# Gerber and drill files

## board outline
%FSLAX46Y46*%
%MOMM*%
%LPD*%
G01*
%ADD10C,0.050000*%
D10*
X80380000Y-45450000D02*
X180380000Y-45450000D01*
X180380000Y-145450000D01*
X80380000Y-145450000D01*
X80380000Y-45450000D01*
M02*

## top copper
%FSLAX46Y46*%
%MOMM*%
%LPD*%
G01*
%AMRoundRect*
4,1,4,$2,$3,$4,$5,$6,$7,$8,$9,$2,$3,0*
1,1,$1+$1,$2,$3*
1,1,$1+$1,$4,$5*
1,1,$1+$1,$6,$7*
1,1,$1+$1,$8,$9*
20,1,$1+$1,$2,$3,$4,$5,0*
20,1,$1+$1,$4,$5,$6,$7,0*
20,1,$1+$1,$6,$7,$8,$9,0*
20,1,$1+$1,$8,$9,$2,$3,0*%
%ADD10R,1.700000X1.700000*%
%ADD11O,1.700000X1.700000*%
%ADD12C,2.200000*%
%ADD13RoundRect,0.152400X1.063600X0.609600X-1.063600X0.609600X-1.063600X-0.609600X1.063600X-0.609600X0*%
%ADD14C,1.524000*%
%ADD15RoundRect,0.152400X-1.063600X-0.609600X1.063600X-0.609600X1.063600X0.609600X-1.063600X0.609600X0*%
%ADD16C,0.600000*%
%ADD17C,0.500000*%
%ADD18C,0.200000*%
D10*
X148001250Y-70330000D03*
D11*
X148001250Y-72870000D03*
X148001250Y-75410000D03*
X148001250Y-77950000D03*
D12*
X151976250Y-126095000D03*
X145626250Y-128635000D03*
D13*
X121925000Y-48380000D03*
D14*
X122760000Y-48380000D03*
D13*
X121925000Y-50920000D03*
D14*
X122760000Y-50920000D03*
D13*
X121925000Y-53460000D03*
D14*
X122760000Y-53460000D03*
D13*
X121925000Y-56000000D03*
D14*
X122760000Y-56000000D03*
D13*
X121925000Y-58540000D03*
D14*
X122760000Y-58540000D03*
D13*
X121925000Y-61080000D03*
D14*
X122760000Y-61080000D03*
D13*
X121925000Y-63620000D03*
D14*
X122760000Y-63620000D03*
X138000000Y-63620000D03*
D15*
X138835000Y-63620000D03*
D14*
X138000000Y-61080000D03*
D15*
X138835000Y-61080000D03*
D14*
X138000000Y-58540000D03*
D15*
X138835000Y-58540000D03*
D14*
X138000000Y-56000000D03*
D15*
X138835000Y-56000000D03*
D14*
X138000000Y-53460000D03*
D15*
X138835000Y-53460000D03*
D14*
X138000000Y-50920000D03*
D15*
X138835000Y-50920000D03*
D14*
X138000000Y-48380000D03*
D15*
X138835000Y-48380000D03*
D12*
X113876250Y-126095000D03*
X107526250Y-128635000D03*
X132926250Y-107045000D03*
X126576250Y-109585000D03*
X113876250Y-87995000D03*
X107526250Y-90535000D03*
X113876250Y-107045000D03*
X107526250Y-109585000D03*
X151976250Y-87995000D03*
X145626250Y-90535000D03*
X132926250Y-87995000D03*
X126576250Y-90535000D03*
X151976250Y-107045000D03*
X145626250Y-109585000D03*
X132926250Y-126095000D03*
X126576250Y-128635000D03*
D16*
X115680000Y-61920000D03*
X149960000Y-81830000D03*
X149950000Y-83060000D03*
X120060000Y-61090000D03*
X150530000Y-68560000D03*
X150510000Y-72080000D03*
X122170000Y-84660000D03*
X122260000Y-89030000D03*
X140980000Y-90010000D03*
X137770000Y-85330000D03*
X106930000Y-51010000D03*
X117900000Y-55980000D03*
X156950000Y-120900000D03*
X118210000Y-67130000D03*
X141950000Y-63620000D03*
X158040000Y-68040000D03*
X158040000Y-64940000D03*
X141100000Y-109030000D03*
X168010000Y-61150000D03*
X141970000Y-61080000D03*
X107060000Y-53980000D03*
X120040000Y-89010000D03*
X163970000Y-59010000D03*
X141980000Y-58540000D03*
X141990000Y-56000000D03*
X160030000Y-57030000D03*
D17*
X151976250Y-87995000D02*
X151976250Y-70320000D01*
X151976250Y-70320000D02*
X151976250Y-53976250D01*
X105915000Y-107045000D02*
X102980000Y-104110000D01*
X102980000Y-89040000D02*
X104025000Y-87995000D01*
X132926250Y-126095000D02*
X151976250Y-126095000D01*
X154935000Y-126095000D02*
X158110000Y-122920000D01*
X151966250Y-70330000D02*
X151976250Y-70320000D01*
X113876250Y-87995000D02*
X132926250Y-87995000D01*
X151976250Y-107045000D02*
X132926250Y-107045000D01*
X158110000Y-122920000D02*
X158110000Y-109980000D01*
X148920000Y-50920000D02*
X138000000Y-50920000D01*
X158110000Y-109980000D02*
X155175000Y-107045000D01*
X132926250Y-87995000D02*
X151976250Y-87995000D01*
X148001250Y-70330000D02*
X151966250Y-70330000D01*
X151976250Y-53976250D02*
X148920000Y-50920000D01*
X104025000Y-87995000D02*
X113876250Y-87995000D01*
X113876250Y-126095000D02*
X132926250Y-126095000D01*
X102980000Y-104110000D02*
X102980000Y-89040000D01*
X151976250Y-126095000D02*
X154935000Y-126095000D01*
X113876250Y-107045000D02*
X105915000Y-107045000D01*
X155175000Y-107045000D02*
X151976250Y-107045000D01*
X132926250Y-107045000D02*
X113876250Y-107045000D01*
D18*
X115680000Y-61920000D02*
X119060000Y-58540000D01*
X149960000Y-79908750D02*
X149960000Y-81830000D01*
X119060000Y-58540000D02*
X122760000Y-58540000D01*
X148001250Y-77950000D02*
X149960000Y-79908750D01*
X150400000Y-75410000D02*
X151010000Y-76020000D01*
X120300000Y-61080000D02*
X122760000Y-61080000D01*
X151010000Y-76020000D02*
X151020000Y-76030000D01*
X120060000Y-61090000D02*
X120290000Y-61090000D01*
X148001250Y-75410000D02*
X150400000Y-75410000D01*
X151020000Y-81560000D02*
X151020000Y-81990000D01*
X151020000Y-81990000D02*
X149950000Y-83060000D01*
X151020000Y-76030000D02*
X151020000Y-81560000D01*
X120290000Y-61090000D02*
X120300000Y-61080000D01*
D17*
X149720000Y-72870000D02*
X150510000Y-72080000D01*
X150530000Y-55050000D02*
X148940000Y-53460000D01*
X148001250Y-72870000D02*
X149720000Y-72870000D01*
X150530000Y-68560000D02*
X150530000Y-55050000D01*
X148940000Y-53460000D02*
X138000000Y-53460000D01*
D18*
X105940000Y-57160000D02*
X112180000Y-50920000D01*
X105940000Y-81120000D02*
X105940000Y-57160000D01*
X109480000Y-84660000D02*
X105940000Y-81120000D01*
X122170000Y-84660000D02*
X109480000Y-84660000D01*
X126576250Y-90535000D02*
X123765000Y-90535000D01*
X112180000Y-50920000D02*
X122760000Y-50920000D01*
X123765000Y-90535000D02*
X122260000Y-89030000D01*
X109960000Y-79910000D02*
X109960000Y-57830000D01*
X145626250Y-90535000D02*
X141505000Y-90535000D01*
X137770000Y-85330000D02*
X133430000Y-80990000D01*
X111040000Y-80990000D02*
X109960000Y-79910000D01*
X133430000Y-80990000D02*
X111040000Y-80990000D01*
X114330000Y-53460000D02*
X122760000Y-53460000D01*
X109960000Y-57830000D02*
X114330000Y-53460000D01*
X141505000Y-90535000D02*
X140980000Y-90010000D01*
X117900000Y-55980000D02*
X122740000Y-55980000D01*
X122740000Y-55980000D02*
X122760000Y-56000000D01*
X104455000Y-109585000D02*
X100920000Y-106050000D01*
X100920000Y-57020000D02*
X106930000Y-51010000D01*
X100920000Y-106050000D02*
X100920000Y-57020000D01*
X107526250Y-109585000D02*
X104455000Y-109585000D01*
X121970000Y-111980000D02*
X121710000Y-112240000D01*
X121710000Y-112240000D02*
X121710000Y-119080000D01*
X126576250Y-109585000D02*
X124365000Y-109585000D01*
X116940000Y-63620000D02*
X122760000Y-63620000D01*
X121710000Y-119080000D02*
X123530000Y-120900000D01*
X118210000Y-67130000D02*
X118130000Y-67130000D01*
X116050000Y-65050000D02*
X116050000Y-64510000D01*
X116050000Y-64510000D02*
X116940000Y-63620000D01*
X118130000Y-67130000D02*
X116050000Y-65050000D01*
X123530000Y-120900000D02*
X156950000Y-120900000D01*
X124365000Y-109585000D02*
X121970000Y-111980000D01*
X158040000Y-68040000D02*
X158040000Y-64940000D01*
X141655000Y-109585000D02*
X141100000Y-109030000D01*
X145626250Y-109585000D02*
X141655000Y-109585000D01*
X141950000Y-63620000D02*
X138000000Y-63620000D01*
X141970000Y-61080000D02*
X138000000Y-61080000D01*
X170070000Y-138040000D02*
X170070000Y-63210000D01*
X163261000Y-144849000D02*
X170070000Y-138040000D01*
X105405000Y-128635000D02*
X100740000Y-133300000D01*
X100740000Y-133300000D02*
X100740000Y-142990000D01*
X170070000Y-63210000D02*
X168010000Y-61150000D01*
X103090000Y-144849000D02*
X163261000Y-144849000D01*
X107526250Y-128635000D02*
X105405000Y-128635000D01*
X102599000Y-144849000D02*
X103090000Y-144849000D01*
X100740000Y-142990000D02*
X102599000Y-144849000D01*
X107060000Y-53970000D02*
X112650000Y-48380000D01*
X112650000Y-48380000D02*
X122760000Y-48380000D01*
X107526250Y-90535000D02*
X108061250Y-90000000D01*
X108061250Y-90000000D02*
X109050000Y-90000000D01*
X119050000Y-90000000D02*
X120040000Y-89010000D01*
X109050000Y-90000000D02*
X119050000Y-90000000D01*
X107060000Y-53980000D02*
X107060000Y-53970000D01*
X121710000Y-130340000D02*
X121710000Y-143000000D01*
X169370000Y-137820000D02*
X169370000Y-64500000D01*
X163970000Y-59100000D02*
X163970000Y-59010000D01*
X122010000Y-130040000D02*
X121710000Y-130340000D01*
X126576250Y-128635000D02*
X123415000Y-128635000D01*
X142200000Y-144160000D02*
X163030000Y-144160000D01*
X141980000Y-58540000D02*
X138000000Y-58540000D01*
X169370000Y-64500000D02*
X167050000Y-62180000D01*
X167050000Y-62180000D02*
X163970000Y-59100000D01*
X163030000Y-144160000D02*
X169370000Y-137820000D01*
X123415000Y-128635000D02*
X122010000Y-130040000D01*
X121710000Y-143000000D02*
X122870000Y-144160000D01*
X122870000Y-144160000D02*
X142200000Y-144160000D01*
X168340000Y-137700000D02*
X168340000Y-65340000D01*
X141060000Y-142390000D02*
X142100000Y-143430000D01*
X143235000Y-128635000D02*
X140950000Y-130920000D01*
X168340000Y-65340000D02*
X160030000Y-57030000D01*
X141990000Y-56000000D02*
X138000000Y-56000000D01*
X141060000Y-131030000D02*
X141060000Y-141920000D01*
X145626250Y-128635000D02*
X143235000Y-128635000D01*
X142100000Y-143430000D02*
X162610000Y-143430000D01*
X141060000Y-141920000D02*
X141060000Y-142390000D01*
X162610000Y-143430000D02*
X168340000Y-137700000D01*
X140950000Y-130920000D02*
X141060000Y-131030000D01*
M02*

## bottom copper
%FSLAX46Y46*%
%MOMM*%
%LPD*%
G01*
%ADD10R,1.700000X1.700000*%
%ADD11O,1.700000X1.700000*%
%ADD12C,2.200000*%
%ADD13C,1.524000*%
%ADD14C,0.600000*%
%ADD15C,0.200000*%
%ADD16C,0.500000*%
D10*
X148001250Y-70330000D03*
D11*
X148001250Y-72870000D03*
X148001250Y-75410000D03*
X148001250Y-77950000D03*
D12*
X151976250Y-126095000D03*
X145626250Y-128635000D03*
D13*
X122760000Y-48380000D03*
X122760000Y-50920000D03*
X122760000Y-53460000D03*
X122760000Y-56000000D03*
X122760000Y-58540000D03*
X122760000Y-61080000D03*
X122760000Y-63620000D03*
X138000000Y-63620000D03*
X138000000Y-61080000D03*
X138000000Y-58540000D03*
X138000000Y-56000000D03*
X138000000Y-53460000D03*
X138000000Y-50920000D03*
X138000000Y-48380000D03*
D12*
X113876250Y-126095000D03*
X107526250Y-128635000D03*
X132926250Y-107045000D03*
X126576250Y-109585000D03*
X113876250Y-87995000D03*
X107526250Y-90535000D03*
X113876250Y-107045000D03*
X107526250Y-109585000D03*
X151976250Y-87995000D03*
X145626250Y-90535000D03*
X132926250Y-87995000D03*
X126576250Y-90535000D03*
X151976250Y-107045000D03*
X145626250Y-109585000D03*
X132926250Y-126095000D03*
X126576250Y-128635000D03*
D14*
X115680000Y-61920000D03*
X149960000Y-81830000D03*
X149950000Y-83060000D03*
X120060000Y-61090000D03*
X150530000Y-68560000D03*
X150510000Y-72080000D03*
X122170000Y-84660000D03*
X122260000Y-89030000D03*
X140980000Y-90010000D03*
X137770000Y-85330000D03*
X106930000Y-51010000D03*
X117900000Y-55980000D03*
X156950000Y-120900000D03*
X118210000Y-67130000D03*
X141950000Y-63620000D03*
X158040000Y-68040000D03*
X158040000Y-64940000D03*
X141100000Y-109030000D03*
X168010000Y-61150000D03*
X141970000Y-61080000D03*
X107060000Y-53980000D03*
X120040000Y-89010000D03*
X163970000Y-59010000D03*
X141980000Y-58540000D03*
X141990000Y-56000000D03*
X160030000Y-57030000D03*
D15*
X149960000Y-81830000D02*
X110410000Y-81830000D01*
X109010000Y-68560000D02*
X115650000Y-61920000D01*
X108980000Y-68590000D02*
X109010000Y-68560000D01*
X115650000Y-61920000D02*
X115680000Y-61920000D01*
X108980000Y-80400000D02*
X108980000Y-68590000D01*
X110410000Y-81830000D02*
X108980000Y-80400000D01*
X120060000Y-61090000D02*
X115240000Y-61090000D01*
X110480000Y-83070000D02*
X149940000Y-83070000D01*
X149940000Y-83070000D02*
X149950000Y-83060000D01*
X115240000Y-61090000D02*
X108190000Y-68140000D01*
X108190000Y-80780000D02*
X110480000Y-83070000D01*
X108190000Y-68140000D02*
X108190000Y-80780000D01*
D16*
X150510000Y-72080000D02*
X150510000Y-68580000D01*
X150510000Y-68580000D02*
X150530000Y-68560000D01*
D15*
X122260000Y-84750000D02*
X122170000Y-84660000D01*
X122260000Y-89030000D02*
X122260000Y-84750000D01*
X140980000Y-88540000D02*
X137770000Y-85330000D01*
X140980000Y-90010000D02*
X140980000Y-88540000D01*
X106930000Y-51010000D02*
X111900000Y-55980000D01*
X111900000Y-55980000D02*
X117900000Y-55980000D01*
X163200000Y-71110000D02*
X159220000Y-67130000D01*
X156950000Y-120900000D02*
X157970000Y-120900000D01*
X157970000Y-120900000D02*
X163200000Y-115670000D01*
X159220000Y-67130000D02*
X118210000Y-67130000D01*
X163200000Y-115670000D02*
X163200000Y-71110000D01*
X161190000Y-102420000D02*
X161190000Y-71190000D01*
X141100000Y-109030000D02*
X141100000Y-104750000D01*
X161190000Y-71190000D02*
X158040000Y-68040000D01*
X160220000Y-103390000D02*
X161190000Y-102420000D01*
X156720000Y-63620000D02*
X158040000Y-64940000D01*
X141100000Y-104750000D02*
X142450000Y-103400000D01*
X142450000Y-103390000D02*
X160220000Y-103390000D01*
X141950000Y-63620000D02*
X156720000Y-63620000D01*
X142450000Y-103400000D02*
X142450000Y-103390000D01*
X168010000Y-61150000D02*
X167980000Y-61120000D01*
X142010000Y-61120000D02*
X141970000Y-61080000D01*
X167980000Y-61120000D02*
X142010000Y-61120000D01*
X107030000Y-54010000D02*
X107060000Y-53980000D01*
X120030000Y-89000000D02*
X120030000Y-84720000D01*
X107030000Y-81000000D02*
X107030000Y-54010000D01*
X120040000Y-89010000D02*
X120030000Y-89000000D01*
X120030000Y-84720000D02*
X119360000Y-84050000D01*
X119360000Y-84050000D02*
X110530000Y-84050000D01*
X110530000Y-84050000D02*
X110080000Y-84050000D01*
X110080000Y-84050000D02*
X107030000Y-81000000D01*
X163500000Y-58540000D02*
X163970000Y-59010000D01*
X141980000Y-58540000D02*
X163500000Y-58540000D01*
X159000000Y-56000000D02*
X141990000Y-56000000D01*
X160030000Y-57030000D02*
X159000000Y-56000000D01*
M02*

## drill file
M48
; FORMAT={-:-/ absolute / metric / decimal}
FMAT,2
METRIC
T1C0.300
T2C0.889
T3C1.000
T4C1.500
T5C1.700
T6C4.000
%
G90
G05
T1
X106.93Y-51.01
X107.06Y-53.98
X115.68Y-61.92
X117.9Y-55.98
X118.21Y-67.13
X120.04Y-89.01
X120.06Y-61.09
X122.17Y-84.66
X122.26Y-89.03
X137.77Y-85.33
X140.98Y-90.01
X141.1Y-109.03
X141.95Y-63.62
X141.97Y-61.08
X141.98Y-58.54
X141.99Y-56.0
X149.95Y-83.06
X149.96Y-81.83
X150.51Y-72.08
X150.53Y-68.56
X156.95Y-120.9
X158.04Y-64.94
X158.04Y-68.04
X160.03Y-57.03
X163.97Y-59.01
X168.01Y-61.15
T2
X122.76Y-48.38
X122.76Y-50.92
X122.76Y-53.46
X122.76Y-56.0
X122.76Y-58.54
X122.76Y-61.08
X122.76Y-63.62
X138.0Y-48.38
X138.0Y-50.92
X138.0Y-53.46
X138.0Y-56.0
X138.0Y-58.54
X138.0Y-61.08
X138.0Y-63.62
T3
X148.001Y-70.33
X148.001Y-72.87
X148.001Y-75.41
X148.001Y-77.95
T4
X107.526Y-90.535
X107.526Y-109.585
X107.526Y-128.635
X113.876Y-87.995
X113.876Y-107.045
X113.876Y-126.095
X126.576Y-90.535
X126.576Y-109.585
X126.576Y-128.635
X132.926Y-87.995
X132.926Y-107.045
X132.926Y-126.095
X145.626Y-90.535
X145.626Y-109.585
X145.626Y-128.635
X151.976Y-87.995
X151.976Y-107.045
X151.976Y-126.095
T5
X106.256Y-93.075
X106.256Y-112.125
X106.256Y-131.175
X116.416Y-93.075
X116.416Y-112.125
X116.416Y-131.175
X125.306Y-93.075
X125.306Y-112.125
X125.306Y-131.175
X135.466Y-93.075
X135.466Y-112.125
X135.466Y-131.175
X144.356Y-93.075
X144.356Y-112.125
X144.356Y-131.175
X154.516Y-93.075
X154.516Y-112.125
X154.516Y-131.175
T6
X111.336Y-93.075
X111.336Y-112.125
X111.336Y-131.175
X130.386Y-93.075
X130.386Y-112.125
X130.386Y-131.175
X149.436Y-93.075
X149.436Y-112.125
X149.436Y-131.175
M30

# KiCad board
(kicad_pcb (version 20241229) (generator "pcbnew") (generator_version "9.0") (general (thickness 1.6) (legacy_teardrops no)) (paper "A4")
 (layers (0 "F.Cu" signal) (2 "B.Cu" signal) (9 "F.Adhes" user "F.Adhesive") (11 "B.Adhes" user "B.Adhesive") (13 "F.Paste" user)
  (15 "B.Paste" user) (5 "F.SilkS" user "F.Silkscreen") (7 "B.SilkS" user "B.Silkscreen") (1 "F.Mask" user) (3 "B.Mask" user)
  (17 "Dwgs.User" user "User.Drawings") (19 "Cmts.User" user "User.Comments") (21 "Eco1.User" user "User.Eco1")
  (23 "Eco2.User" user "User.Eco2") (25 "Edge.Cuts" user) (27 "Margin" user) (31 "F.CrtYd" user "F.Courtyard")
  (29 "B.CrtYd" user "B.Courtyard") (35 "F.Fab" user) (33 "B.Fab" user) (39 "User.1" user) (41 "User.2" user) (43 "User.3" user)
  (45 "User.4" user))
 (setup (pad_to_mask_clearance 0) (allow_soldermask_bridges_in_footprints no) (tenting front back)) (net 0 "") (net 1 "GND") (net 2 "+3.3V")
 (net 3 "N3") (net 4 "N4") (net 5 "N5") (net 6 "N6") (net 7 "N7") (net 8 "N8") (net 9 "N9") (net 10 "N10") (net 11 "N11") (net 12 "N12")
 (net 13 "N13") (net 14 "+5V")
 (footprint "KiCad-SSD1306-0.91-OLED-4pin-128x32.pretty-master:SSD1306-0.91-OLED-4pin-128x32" (layer "F.Cu") (at 111.50125 68.14)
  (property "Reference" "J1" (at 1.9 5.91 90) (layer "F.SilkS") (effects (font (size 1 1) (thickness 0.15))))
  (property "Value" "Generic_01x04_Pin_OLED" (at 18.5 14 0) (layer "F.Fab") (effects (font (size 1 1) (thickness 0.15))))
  (pad "1" thru_hole rect (at 36.5 2.19) (size 1.7 1.7) (drill 1) (layers "*.Cu" "*.Mask") (remove_unused_layers no) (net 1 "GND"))
  (pad "2" thru_hole oval (at 36.5 4.73) (size 1.7 1.7) (drill 1) (layers "*.Cu" "*.Mask") (remove_unused_layers no) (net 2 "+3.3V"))
  (pad "3" thru_hole oval (at 36.5 7.27) (size 1.7 1.7) (drill 1) (layers "*.Cu" "*.Mask") (remove_unused_layers no) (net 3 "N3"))
  (pad "4" thru_hole oval (at 36.5 9.81) (size 1.7 1.7) (drill 1) (layers "*.Cu" "*.Mask") (remove_unused_layers no) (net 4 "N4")))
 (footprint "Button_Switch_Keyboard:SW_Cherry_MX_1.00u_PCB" (layer "F.Cu") (at 151.97625 126.095)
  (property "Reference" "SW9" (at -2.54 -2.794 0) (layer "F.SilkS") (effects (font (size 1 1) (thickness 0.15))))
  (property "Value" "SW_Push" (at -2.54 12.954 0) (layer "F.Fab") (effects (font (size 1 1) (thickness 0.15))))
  (pad "" np_thru_hole circle (at -7.62 5.08) (size 1.7 1.7) (drill 1.7) (layers "*.Cu" "*.Mask"))
  (pad "" np_thru_hole circle (at -2.54 5.08) (size 4 4) (drill 4) (layers "*.Cu" "*.Mask"))
  (pad "" np_thru_hole circle (at 2.54 5.08) (size 1.7 1.7) (drill 1.7) (layers "*.Cu" "*.Mask"))
  (pad "1" thru_hole circle (at 0 0) (size 2.2 2.2) (drill 1.5) (layers "*.Cu" "*.Mask") (remove_unused_layers no) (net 1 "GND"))
  (pad "2" thru_hole circle (at -6.35 2.54) (size 2.2 2.2) (drill 1.5) (layers "*.Cu" "*.Mask") (remove_unused_layers no) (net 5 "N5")))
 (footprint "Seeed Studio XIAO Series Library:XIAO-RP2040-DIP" (layer "F.Cu") (at 130.38 56)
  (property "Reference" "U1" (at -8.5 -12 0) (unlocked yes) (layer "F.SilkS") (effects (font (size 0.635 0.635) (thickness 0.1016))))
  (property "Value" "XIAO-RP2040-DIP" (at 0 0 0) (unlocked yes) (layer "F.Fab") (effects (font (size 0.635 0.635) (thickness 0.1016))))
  (pad "1" smd roundrect (at -8.455 -7.62 180) (size 2.432 1.524) (layers "F.Cu" "F.Mask") (roundrect_rratio 0.1) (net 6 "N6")
   (thermal_bridge_angle 45))
  (pad "1" thru_hole circle (at -7.62 -7.62 180) (size 1.524 1.524) (drill 0.889) (layers "*.Cu" "*.Mask") (remove_unused_layers no)
   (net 6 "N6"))
  (pad "2" smd roundrect (at -8.455 -5.08 180) (size 2.432 1.524) (layers "F.Cu" "F.Mask") (roundrect_rratio 0.1) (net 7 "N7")
   (thermal_bridge_angle 45))
  (pad "2" thru_hole circle (at -7.62 -5.08 180) (size 1.524 1.524) (drill 0.889) (layers "*.Cu" "*.Mask") (remove_unused_layers no)
   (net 7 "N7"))
  (pad "3" smd roundrect (at -8.455 -2.54 180) (size 2.432 1.524) (layers "F.Cu" "F.Mask") (roundrect_rratio 0.1) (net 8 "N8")
   (thermal_bridge_angle 45))
  (pad "3" thru_hole circle (at -7.62 -2.54 180) (size 1.524 1.524) (drill 0.889) (layers "*.Cu" "*.Mask") (remove_unused_layers no)
   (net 8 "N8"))
  (pad "4" smd roundrect (at -8.455 0 180) (size 2.432 1.524) (layers "F.Cu" "F.Mask") (roundrect_rratio 0.1) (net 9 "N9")
   (thermal_bridge_angle 45))
  (pad "4" thru_hole circle (at -7.62 0 180) (size 1.524 1.524) (drill 0.889) (layers "*.Cu" "*.Mask") (remove_unused_layers no)
   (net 9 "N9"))
  (pad "5" smd roundrect (at -8.455 2.54 180) (size 2.432 1.524) (layers "F.Cu" "F.Mask") (roundrect_rratio 0.1) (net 4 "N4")
   (thermal_bridge_angle 45))
  (pad "5" thru_hole circle (at -7.62 2.54 180) (size 1.524 1.524) (drill 0.889) (layers "*.Cu" "*.Mask") (remove_unused_layers no)
   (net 4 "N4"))
  (pad "6" smd roundrect (at -8.455 5.08 180) (size 2.432 1.524) (layers "F.Cu" "F.Mask") (roundrect_rratio 0.1) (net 3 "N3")
   (thermal_bridge_angle 45))
  (pad "6" thru_hole circle (at -7.62 5.08 180) (size 1.524 1.524) (drill 0.889) (layers "*.Cu" "*.Mask") (remove_unused_layers no)
   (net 3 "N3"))
  (pad "7" smd roundrect (at -8.455 7.62 180) (size 2.432 1.524) (layers "F.Cu" "F.Mask") (roundrect_rratio 0.1) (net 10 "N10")
   (thermal_bridge_angle 45))
  (pad "7" thru_hole circle (at -7.62 7.62 180) (size 1.524 1.524) (drill 0.889) (layers "*.Cu" "*.Mask") (remove_unused_layers no)
   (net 10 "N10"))
  (pad "8" thru_hole circle (at 7.62 7.62) (size 1.524 1.524) (drill 0.889) (layers "*.Cu" "*.Mask") (remove_unused_layers no)
   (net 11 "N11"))
  (pad "8" smd roundrect (at 8.455 7.62) (size 2.432 1.524) (layers "F.Cu" "F.Mask") (roundrect_rratio 0.1) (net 11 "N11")
   (thermal_bridge_angle 45))
  (pad "9" thru_hole circle (at 7.62 5.08) (size 1.524 1.524) (drill 0.889) (layers "*.Cu" "*.Mask") (remove_unused_layers no)
   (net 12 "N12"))
  (pad "9" smd roundrect (at 8.455 5.08) (size 2.432 1.524) (layers "F.Cu" "F.Mask") (roundrect_rratio 0.1) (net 12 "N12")
   (thermal_bridge_angle 45))
  (pad "10" thru_hole circle (at 7.62 2.54) (size 1.524 1.524) (drill 0.889) (layers "*.Cu" "*.Mask") (remove_unused_layers no)
   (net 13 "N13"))
  (pad "10" smd roundrect (at 8.455 2.54) (size 2.432 1.524) (layers "F.Cu" "F.Mask") (roundrect_rratio 0.1) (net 13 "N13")
   (thermal_bridge_angle 45))
  (pad "11" thru_hole circle (at 7.62 0) (size 1.524 1.524) (drill 0.889) (layers "*.Cu" "*.Mask") (remove_unused_layers no) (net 5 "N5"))
  (pad "11" smd roundrect (at 8.455 0) (size 2.432 1.524) (layers "F.Cu" "F.Mask") (roundrect_rratio 0.1) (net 5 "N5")
   (thermal_bridge_angle 45))
  (pad "12" thru_hole circle (at 7.62 -2.54) (size 1.524 1.524) (drill 0.889) (layers "*.Cu" "*.Mask") (remove_unused_layers no)
   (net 2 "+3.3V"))
  (pad "12" smd roundrect (at 8.455 -2.54) (size 2.432 1.524) (layers "F.Cu" "F.Mask") (roundrect_rratio 0.1) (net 2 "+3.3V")
   (thermal_bridge_angle 45))
  (pad "13" thru_hole circle (at 7.62 -5.08) (size 1.524 1.524) (drill 0.889) (layers "*.Cu" "*.Mask") (remove_unused_layers no)
   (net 1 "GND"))
  (pad "13" smd roundrect (at 8.455 -5.08) (size 2.432 1.524) (layers "F.Cu" "F.Mask") (roundrect_rratio 0.1) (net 1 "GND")
   (thermal_bridge_angle 45))
  (pad "14" thru_hole circle (at 7.62 -7.62) (size 1.524 1.524) (drill 0.889) (layers "*.Cu" "*.Mask") (remove_unused_layers no)
   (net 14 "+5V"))
  (pad "14" smd roundrect (at 8.455 -7.62) (size 2.432 1.524) (layers "F.Cu" "F.Mask") (roundrect_rratio 0.1) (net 14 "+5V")
   (thermal_bridge_angle 45)))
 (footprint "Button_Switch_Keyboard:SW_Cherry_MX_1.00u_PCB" (layer "F.Cu") (at 113.87625 126.095)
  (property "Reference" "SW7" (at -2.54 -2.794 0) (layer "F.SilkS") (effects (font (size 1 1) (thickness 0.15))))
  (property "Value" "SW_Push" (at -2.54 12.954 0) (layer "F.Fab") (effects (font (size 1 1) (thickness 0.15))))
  (pad "" np_thru_hole circle (at -7.62 5.08) (size 1.7 1.7) (drill 1.7) (layers "*.Cu" "*.Mask"))
  (pad "" np_thru_hole circle (at -2.54 5.08) (size 4 4) (drill 4) (layers "*.Cu" "*.Mask"))
  (pad "" np_thru_hole circle (at 2.54 5.08) (size 1.7 1.7) (drill 1.7) (layers "*.Cu" "*.Mask"))
  (pad "1" thru_hole circle (at 0 0) (size 2.2 2.2) (drill 1.5) (layers "*.Cu" "*.Mask") (remove_unused_layers no) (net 1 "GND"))
  (pad "2" thru_hole circle (at -6.35 2.54) (size 2.2 2.2) (drill 1.5) (layers "*.Cu" "*.Mask") (remove_unused_layers no) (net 12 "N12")))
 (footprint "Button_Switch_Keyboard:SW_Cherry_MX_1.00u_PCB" (layer "F.Cu") (at 132.92625 107.045)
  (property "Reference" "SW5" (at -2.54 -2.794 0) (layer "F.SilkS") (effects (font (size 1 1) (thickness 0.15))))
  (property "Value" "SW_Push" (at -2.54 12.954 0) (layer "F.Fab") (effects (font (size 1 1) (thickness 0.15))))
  (pad "" np_thru_hole circle (at -7.62 5.08) (size 1.7 1.7) (drill 1.7) (layers "*.Cu" "*.Mask"))
  (pad "" np_thru_hole circle (at -2.54 5.08) (size 4 4) (drill 4) (layers "*.Cu" "*.Mask"))
  (pad "" np_thru_hole circle (at 2.54 5.08) (size 1.7 1.7) (drill 1.7) (layers "*.Cu" "*.Mask"))
  (pad "1" thru_hole circle (at 0 0) (size 2.2 2.2) (drill 1.5) (layers "*.Cu" "*.Mask") (remove_unused_layers no) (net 1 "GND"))
  (pad "2" thru_hole circle (at -6.35 2.54) (size 2.2 2.2) (drill 1.5) (layers "*.Cu" "*.Mask") (remove_unused_layers no) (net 10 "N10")))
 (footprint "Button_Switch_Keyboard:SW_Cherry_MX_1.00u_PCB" (layer "F.Cu") (at 113.87625 87.995)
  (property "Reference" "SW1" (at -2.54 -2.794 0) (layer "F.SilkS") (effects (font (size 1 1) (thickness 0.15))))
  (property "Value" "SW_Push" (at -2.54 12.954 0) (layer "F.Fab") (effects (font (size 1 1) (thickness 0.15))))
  (pad "" np_thru_hole circle (at -7.62 5.08) (size 1.7 1.7) (drill 1.7) (layers "*.Cu" "*.Mask"))
  (pad "" np_thru_hole circle (at -2.54 5.08) (size 4 4) (drill 4) (layers "*.Cu" "*.Mask"))
  (pad "" np_thru_hole circle (at 2.54 5.08) (size 1.7 1.7) (drill 1.7) (layers "*.Cu" "*.Mask"))
  (pad "1" thru_hole circle (at 0 0) (size 2.2 2.2) (drill 1.5) (layers "*.Cu" "*.Mask") (remove_unused_layers no) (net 1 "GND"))
  (pad "2" thru_hole circle (at -6.35 2.54) (size 2.2 2.2) (drill 1.5) (layers "*.Cu" "*.Mask") (remove_unused_layers no) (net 6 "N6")))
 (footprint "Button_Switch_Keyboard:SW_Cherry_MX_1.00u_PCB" (layer "F.Cu") (at 113.87625 107.045)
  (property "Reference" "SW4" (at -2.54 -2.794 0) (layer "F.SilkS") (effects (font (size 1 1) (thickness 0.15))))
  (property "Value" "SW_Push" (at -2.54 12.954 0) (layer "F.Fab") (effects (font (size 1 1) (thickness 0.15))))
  (pad "" np_thru_hole circle (at -7.62 5.08) (size 1.7 1.7) (drill 1.7) (layers "*.Cu" "*.Mask"))
  (pad "" np_thru_hole circle (at -2.54 5.08) (size 4 4) (drill 4) (layers "*.Cu" "*.Mask"))
  (pad "" np_thru_hole circle (at 2.54 5.08) (size 1.7 1.7) (drill 1.7) (layers "*.Cu" "*.Mask"))
  (pad "1" thru_hole circle (at 0 0) (size 2.2 2.2) (drill 1.5) (layers "*.Cu" "*.Mask") (remove_unused_layers no) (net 1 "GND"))
  (pad "2" thru_hole circle (at -6.35 2.54) (size 2.2 2.2) (drill 1.5) (layers "*.Cu" "*.Mask") (remove_unused_layers no) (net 9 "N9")))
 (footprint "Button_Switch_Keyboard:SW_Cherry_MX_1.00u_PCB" (layer "F.Cu") (at 151.97625 87.995)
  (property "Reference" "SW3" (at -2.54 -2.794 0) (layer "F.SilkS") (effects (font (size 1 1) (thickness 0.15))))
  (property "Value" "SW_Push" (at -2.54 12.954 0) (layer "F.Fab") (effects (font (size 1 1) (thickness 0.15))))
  (pad "" np_thru_hole circle (at -7.62 5.08) (size 1.7 1.7) (drill 1.7) (layers "*.Cu" "*.Mask"))
  (pad "" np_thru_hole circle (at -2.54 5.08) (size 4 4) (drill 4) (layers "*.Cu" "*.Mask"))
  (pad "" np_thru_hole circle (at 2.54 5.08) (size 1.7 1.7) (drill 1.7) (layers "*.Cu" "*.Mask"))
  (pad "1" thru_hole circle (at 0 0) (size 2.2 2.2) (drill 1.5) (layers "*.Cu" "*.Mask") (remove_unused_layers no) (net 1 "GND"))
  (pad "2" thru_hole circle (at -6.35 2.54) (size 2.2 2.2) (drill 1.5) (layers "*.Cu" "*.Mask") (remove_unused_layers no) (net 8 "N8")))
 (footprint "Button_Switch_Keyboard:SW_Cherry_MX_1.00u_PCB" (layer "F.Cu") (at 132.92625 87.995)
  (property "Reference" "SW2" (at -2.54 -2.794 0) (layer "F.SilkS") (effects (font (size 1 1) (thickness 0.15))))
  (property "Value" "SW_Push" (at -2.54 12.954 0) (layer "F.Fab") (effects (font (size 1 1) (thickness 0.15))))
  (pad "" np_thru_hole circle (at -7.62 5.08) (size 1.7 1.7) (drill 1.7) (layers "*.Cu" "*.Mask"))
  (pad "" np_thru_hole circle (at -2.54 5.08) (size 4 4) (drill 4) (layers "*.Cu" "*.Mask"))
  (pad "" np_thru_hole circle (at 2.54 5.08) (size 1.7 1.7) (drill 1.7) (layers "*.Cu" "*.Mask"))
  (pad "1" thru_hole circle (at 0 0) (size 2.2 2.2) (drill 1.5) (layers "*.Cu" "*.Mask") (remove_unused_layers no) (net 1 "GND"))
  (pad "2" thru_hole circle (at -6.35 2.54) (size 2.2 2.2) (drill 1.5) (layers "*.Cu" "*.Mask") (remove_unused_layers no) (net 7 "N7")))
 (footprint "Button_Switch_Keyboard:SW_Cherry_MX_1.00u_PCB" (layer "F.Cu") (at 151.97625 107.045)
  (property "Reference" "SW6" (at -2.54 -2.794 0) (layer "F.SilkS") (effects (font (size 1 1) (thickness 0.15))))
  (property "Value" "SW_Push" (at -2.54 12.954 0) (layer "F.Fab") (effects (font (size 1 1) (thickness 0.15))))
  (pad "" np_thru_hole circle (at -7.62 5.08) (size 1.7 1.7) (drill 1.7) (layers "*.Cu" "*.Mask"))
  (pad "" np_thru_hole circle (at -2.54 5.08) (size 4 4) (drill 4) (layers "*.Cu" "*.Mask"))
  (pad "" np_thru_hole circle (at 2.54 5.08) (size 1.7 1.7) (drill 1.7) (layers "*.Cu" "*.Mask"))
  (pad "1" thru_hole circle (at 0 0) (size 2.2 2.2) (drill 1.5) (layers "*.Cu" "*.Mask") (remove_unused_layers no) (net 1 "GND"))
  (pad "2" thru_hole circle (at -6.35 2.54) (size 2.2 2.2) (drill 1.5) (layers "*.Cu" "*.Mask") (remove_unused_layers no) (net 11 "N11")))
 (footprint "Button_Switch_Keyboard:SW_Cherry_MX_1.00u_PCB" (layer "F.Cu") (at 132.92625 126.095)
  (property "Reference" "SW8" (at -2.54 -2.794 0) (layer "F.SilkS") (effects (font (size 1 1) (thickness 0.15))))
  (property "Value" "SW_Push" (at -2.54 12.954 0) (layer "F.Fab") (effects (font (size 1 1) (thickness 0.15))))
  (pad "" np_thru_hole circle (at -7.62 5.08) (size 1.7 1.7) (drill 1.7) (layers "*.Cu" "*.Mask"))
  (pad "" np_thru_hole circle (at -2.54 5.08) (size 4 4) (drill 4) (layers "*.Cu" "*.Mask"))
  (pad "" np_thru_hole circle (at 2.54 5.08) (size 1.7 1.7) (drill 1.7) (layers "*.Cu" "*.Mask"))
  (pad "1" thru_hole circle (at 0 0) (size 2.2 2.2) (drill 1.5) (layers "*.Cu" "*.Mask") (remove_unused_layers no) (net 1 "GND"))
  (pad "2" thru_hole circle (at -6.35 2.54) (size 2.2 2.2) (drill 1.5) (layers "*.Cu" "*.Mask") (remove_unused_layers no) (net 13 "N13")))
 (gr_rect (start 80.38 45.45) (end 180.38 145.45) (stroke (width 0.05) (type default)) (fill no) (layer "Edge.Cuts"))
 (segment (start 151.97625 87.995) (end 151.97625 70.32) (width 0.5) (layer "F.Cu") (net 1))
 (segment (start 151.97625 70.32) (end 151.97625 53.97625) (width 0.5) (layer "F.Cu") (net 1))
 (segment (start 105.915 107.045) (end 102.98 104.11) (width 0.5) (layer "F.Cu") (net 1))
 (segment (start 102.98 89.04) (end 104.025 87.995) (width 0.5) (layer "F.Cu") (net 1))
 (segment (start 132.92625 126.095) (end 151.97625 126.095) (width 0.5) (layer "F.Cu") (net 1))
 (segment (start 154.935 126.095) (end 158.11 122.92) (width 0.5) (layer "F.Cu") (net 1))
 (segment (start 151.96625 70.33) (end 151.97625 70.32) (width 0.5) (layer "F.Cu") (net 1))
 (segment (start 113.87625 87.995) (end 132.92625 87.995) (width 0.5) (layer "F.Cu") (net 1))
 (segment (start 151.97625 107.045) (end 132.92625 107.045) (width 0.5) (layer "F.Cu") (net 1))
 (segment (start 158.11 122.92) (end 158.11 109.98) (width 0.5) (layer "F.Cu") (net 1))
 (segment (start 148.92 50.92) (end 138 50.92) (width 0.5) (layer "F.Cu") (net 1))
 (segment (start 158.11 109.98) (end 155.175 107.045) (width 0.5) (layer "F.Cu") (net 1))
 (segment (start 132.92625 87.995) (end 151.97625 87.995) (width 0.5) (layer "F.Cu") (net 1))
 (segment (start 148.00125 70.33) (end 151.96625 70.33) (width 0.5) (layer "F.Cu") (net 1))
 (segment (start 151.97625 53.97625) (end 148.92 50.92) (width 0.5) (layer "F.Cu") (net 1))
 (segment (start 104.025 87.995) (end 113.87625 87.995) (width 0.5) (layer "F.Cu") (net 1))
 (segment (start 113.87625 126.095) (end 132.92625 126.095) (width 0.5) (layer "F.Cu") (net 1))
 (segment (start 102.98 104.11) (end 102.98 89.04) (width 0.5) (layer "F.Cu") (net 1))
 (segment (start 151.97625 126.095) (end 154.935 126.095) (width 0.5) (layer "F.Cu") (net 1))
 (segment (start 113.87625 107.045) (end 105.915 107.045) (width 0.5) (layer "F.Cu") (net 1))
 (segment (start 155.175 107.045) (end 151.97625 107.045) (width 0.5) (layer "F.Cu") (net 1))
 (segment (start 132.92625 107.045) (end 113.87625 107.045) (width 0.5) (layer "F.Cu") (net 1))
 (segment (start 115.68 61.92) (end 119.06 58.54) (width 0.2) (layer "F.Cu") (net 4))
 (segment (start 149.96 79.90875) (end 149.96 81.83) (width 0.2) (layer "F.Cu") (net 4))
 (segment (start 119.06 58.54) (end 122.76 58.54) (width 0.2) (layer "F.Cu") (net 4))
 (segment (start 148.00125 77.95) (end 149.96 79.90875) (width 0.2) (layer "F.Cu") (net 4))
 (via (at 115.68 61.92) (size 0.6) (drill 0.3) (layers "F.Cu" "B.Cu") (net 4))
 (via (at 149.96 81.83) (size 0.6) (drill 0.3) (layers "F.Cu" "B.Cu") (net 4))
 (segment (start 149.96 81.83) (end 110.41 81.83) (width 0.2) (layer "B.Cu") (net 4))
 (segment (start 109.01 68.56) (end 115.65 61.92) (width 0.2) (layer "B.Cu") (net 4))
 (segment (start 108.98 68.59) (end 109.01 68.56) (width 0.2) (layer "B.Cu") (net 4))
 (segment (start 115.65 61.92) (end 115.68 61.92) (width 0.2) (layer "B.Cu") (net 4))
 (segment (start 108.98 80.4) (end 108.98 68.59) (width 0.2) (layer "B.Cu") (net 4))
 (segment (start 110.41 81.83) (end 108.98 80.4) (width 0.2) (layer "B.Cu") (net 4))
 (segment (start 150.4 75.41) (end 151.01 76.02) (width 0.2) (layer "F.Cu") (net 3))
 (segment (start 120.3 61.08) (end 122.76 61.08) (width 0.2) (layer "F.Cu") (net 3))
 (segment (start 151.01 76.02) (end 151.02 76.03) (width 0.2) (layer "F.Cu") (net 3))
 (segment (start 120.06 61.09) (end 120.29 61.09) (width 0.2) (layer "F.Cu") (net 3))
 (segment (start 148.00125 75.41) (end 150.4 75.41) (width 0.2) (layer "F.Cu") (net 3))
 (segment (start 151.02 81.56) (end 151.02 81.99) (width 0.2) (layer "F.Cu") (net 3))
 (segment (start 151.02 81.99) (end 149.95 83.06) (width 0.2) (layer "F.Cu") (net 3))
 (segment (start 151.02 76.03) (end 151.02 81.56) (width 0.2) (layer "F.Cu") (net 3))
 (segment (start 120.29 61.09) (end 120.3 61.08) (width 0.2) (layer "F.Cu") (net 3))
 (via (at 149.95 83.06) (size 0.6) (drill 0.3) (layers "F.Cu" "B.Cu") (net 3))
 (via (at 120.06 61.09) (size 0.6) (drill 0.3) (layers "F.Cu" "B.Cu") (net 3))
 (segment (start 120.06 61.09) (end 115.24 61.09) (width 0.2) (layer "B.Cu") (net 3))
 (segment (start 110.48 83.07) (end 149.94 83.07) (width 0.2) (layer "B.Cu") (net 3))
 (segment (start 149.94 83.07) (end 149.95 83.06) (width 0.2) (layer "B.Cu") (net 3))
 (segment (start 115.24 61.09) (end 108.19 68.14) (width 0.2) (layer "B.Cu") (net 3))
 (segment (start 108.19 80.78) (end 110.48 83.07) (width 0.2) (layer "B.Cu") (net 3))
 (segment (start 108.19 68.14) (end 108.19 80.78) (width 0.2) (layer "B.Cu") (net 3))
 (segment (start 149.72 72.87) (end 150.51 72.08) (width 0.5) (layer "F.Cu") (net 2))
 (segment (start 150.53 55.05) (end 148.94 53.46) (width 0.5) (layer "F.Cu") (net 2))
 (segment (start 148.00125 72.87) (end 149.72 72.87) (width 0.5) (layer "F.Cu") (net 2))
 (segment (start 150.53 68.56) (end 150.53 55.05) (width 0.5) (layer "F.Cu") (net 2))
 (segment (start 148.94 53.46) (end 138 53.46) (width 0.5) (layer "F.Cu") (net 2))
 (via (at 150.53 68.56) (size 0.6) (drill 0.3) (layers "F.Cu" "B.Cu") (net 2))
 (via (at 150.51 72.08) (size 0.6) (drill 0.3) (layers "F.Cu" "B.Cu") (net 2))
 (segment (start 150.51 72.08) (end 150.51 68.58) (width 0.5) (layer "B.Cu") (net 2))
 (segment (start 150.51 68.58) (end 150.53 68.56) (width 0.5) (layer "B.Cu") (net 2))
 (segment (start 105.94 57.16) (end 112.18 50.92) (width 0.2) (layer "F.Cu") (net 7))
 (segment (start 105.94 81.12) (end 105.94 57.16) (width 0.2) (layer "F.Cu") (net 7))
 (segment (start 109.48 84.66) (end 105.94 81.12) (width 0.2) (layer "F.Cu") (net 7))
 (segment (start 122.17 84.66) (end 109.48 84.66) (width 0.2) (layer "F.Cu") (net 7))
 (segment (start 126.57625 90.535) (end 123.765 90.535) (width 0.2) (layer "F.Cu") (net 7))
 (segment (start 112.18 50.92) (end 122.76 50.92) (width 0.2) (layer "F.Cu") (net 7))
 (segment (start 123.765 90.535) (end 122.26 89.03) (width 0.2) (layer "F.Cu") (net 7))
 (via (at 122.17 84.66) (size 0.6) (drill 0.3) (layers "F.Cu" "B.Cu") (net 7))
 (via (at 122.26 89.03) (size 0.6) (drill 0.3) (layers "F.Cu" "B.Cu") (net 7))
 (segment (start 122.26 84.75) (end 122.17 84.66) (width 0.2) (layer "B.Cu") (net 7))
 (segment (start 122.26 89.03) (end 122.26 84.75) (width 0.2) (layer "B.Cu") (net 7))
 (segment (start 109.96 79.91) (end 109.96 57.83) (width 0.2) (layer "F.Cu") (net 8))
 (segment (start 145.62625 90.535) (end 141.505 90.535) (width 0.2) (layer "F.Cu") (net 8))
 (segment (start 137.77 85.33) (end 133.43 80.99) (width 0.2) (layer "F.Cu") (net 8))
 (segment (start 111.04 80.99) (end 109.96 79.91) (width 0.2) (layer "F.Cu") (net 8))
 (segment (start 133.43 80.99) (end 111.04 80.99) (width 0.2) (layer "F.Cu") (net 8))
 (segment (start 114.33 53.46) (end 122.76 53.46) (width 0.2) (layer "F.Cu") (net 8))
 (segment (start 109.96 57.83) (end 114.33 53.46) (width 0.2) (layer "F.Cu") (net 8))
 (segment (start 141.505 90.535) (end 140.98 90.01) (width 0.2) (layer "F.Cu") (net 8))
 (via (at 140.98 90.01) (size 0.6) (drill 0.3) (layers "F.Cu" "B.Cu") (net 8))
 (via (at 137.77 85.33) (size 0.6) (drill 0.3) (layers "F.Cu" "B.Cu") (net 8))
 (segment (start 140.98 88.54) (end 137.77 85.33) (width 0.2) (layer "B.Cu") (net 8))
 (segment (start 140.98 90.01) (end 140.98 88.54) (width 0.2) (layer "B.Cu") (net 8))
 (segment (start 117.9 55.98) (end 122.74 55.98) (width 0.2) (layer "F.Cu") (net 9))
 (segment (start 122.74 55.98) (end 122.76 56) (width 0.2) (layer "F.Cu") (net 9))
 (segment (start 104.455 109.585) (end 100.92 106.05) (width 0.2) (layer "F.Cu") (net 9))
 (segment (start 100.92 57.02) (end 106.93 51.01) (width 0.2) (layer "F.Cu") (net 9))
 (segment (start 100.92 106.05) (end 100.92 57.02) (width 0.2) (layer "F.Cu") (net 9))
 (segment (start 107.52625 109.585) (end 104.455 109.585) (width 0.2) (layer "F.Cu") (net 9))
 (via (at 106.93 51.01) (size 0.6) (drill 0.3) (layers "F.Cu" "B.Cu") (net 9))
 (via (at 117.9 55.98) (size 0.6) (drill 0.3) (layers "F.Cu" "B.Cu") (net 9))
 (segment (start 106.93 51.01) (end 111.9 55.98) (width 0.2) (layer "B.Cu") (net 9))
 (segment (start 111.9 55.98) (end 117.9 55.98) (width 0.2) (layer "B.Cu") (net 9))
 (segment (start 121.97 111.98) (end 121.71 112.24) (width 0.2) (layer "F.Cu") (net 10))
 (segment (start 121.71 112.24) (end 121.71 119.08) (width 0.2) (layer "F.Cu") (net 10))
 (segment (start 126.57625 109.585) (end 124.365 109.585) (width 0.2) (layer "F.Cu") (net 10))
 (segment (start 116.94 63.62) (end 122.76 63.62) (width 0.2) (layer "F.Cu") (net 10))
 (segment (start 121.71 119.08) (end 123.53 120.9) (width 0.2) (layer "F.Cu") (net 10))
 (segment (start 118.21 67.13) (end 118.13 67.13) (width 0.2) (layer "F.Cu") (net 10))
 (segment (start 116.05 65.05) (end 116.05 64.51) (width 0.2) (layer "F.Cu") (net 10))
 (segment (start 116.05 64.51) (end 116.94 63.62) (width 0.2) (layer "F.Cu") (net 10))
 (segment (start 118.13 67.13) (end 116.05 65.05) (width 0.2) (layer "F.Cu") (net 10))
 (segment (start 123.53 120.9) (end 156.95 120.9) (width 0.2) (layer "F.Cu") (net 10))
 (segment (start 124.365 109.585) (end 121.97 111.98) (width 0.2) (layer "F.Cu") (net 10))
 (via (at 156.95 120.9) (size 0.6) (drill 0.3) (layers "F.Cu" "B.Cu") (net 10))
 (via (at 118.21 67.13) (size 0.6) (drill 0.3) (layers "F.Cu" "B.Cu") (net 10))
 (segment (start 163.2 71.11) (end 159.22 67.13) (width 0.2) (layer "B.Cu") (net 10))
 (segment (start 156.95 120.9) (end 157.97 120.9) (width 0.2) (layer "B.Cu") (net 10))
 (segment (start 157.97 120.9) (end 163.2 115.67) (width 0.2) (layer "B.Cu") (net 10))
 (segment (start 159.22 67.13) (end 118.21 67.13) (width 0.2) (layer "B.Cu") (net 10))
 (segment (start 163.2 115.67) (end 163.2 71.11) (width 0.2) (layer "B.Cu") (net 10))
 (segment (start 158.04 68.04) (end 158.04 64.94) (width 0.2) (layer "F.Cu") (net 11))
 (segment (start 141.655 109.585) (end 141.1 109.03) (width 0.2) (layer "F.Cu") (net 11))
 (segment (start 145.62625 109.585) (end 141.655 109.585) (width 0.2) (layer "F.Cu") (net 11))
 (segment (start 141.95 63.62) (end 138 63.62) (width 0.2) (layer "F.Cu") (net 11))
 (via (at 141.95 63.62) (size 0.6) (drill 0.3) (layers "F.Cu" "B.Cu") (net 11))
 (via (at 158.04 68.04) (size 0.6) (drill 0.3) (layers "F.Cu" "B.Cu") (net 11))
 (via (at 158.04 64.94) (size 0.6) (drill 0.3) (layers "F.Cu" "B.Cu") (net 11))
 (via (at 141.1 109.03) (size 0.6) (drill 0.3) (layers "F.Cu" "B.Cu") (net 11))
 (segment (start 161.19 102.42) (end 161.19 71.19) (width 0.2) (layer "B.Cu") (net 11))
 (segment (start 141.1 109.03) (end 141.1 104.75) (width 0.2) (layer "B.Cu") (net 11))
 (segment (start 161.19 71.19) (end 158.04 68.04) (width 0.2) (layer "B.Cu") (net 11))
 (segment (start 160.22 103.39) (end 161.19 102.42) (width 0.2) (layer "B.Cu") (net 11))
 (segment (start 156.72 63.62) (end 158.04 64.94) (width 0.2) (layer "B.Cu") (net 11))
 (segment (start 141.1 104.75) (end 142.45 103.4) (width 0.2) (layer "B.Cu") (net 11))
 (segment (start 142.45 103.39) (end 160.22 103.39) (width 0.2) (layer "B.Cu") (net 11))
 (segment (start 141.95 63.62) (end 156.72 63.62) (width 0.2) (layer "B.Cu") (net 11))
 (segment (start 142.45 103.4) (end 142.45 103.39) (width 0.2) (layer "B.Cu") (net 11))
 (segment (start 141.97 61.08) (end 138 61.08) (width 0.2) (layer "F.Cu") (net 12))
 (segment (start 170.07 138.04) (end 170.07 63.21) (width 0.2) (layer "F.Cu") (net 12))
 (segment (start 163.261 144.849) (end 170.07 138.04) (width 0.2) (layer "F.Cu") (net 12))
 (segment (start 105.405 128.635) (end 100.74 133.3) (width 0.2) (layer "F.Cu") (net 12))
 (segment (start 100.74 133.3) (end 100.74 142.99) (width 0.2) (layer "F.Cu") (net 12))
 (segment (start 170.07 63.21) (end 168.01 61.15) (width 0.2) (layer "F.Cu") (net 12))
 (segment (start 103.09 144.849) (end 163.261 144.849) (width 0.2) (layer "F.Cu") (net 12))
 (segment (start 107.52625 128.635) (end 105.405 128.635) (width 0.2) (layer "F.Cu") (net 12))
 (segment (start 102.599 144.849) (end 103.09 144.849) (width 0.2) (layer "F.Cu") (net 12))
 (segment (start 100.74 142.99) (end 102.599 144.849) (width 0.2) (layer "F.Cu") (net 12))
 (via (at 168.01 61.15) (size 0.6) (drill 0.3) (layers "F.Cu" "B.Cu") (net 12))
 (via (at 141.97 61.08) (size 0.6) (drill 0.3) (layers "F.Cu" "B.Cu") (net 12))
 (segment (start 168.01 61.15) (end 167.98 61.12) (width 0.2) (layer "B.Cu") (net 12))
 (segment (start 142.01 61.12) (end 141.97 61.08) (width 0.2) (layer "B.Cu") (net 12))
 (segment (start 167.98 61.12) (end 142.01 61.12) (width 0.2) (layer "B.Cu") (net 12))
 (segment (start 107.06 53.97) (end 112.65 48.38) (width 0.2) (layer "F.Cu") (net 6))
 (segment (start 112.65 48.38) (end 122.76 48.38) (width 0.2) (layer "F.Cu") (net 6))
 (segment (start 107.52625 90.535) (end 108.06125 90) (width 0.2) (layer "F.Cu") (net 6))
 (segment (start 108.06125 90) (end 109.05 90) (width 0.2) (layer "F.Cu") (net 6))
 (segment (start 119.05 90) (end 120.04 89.01) (width 0.2) (layer "F.Cu") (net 6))
 (segment (start 109.05 90) (end 119.05 90) (width 0.2) (layer "F.Cu") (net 6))
 (segment (start 107.06 53.98) (end 107.06 53.97) (width 0.2) (layer "F.Cu") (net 6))
 (via (at 107.06 53.98) (size 0.6) (drill 0.3) (layers "F.Cu" "B.Cu") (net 6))
 (via (at 120.04 89.01) (size 0.6) (drill 0.3) (layers "F.Cu" "B.Cu") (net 6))
 (segment (start 107.03 54.01) (end 107.06 53.98) (width 0.2) (layer "B.Cu") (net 6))
 (segment (start 120.03 89) (end 120.03 84.72) (width 0.2) (layer "B.Cu") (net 6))
 (segment (start 107.03 81) (end 107.03 54.01) (width 0.2) (layer "B.Cu") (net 6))
 (segment (start 120.04 89.01) (end 120.03 89) (width 0.2) (layer "B.Cu") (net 6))
 (segment (start 120.03 84.72) (end 119.36 84.05) (width 0.2) (layer "B.Cu") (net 6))
 (segment (start 119.36 84.05) (end 110.53 84.05) (width 0.2) (layer "B.Cu") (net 6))
 (segment (start 110.53 84.05) (end 110.08 84.05) (width 0.2) (layer "B.Cu") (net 6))
 (segment (start 110.08 84.05) (end 107.03 81) (width 0.2) (layer "B.Cu") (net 6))
 (segment (start 121.71 130.34) (end 121.71 143) (width 0.2) (layer "F.Cu") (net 13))
 (segment (start 169.37 137.82) (end 169.37 64.5) (width 0.2) (layer "F.Cu") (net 13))
 (segment (start 163.97 59.1) (end 163.97 59.01) (width 0.2) (layer "F.Cu") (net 13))
 (segment (start 122.01 130.04) (end 121.71 130.34) (width 0.2) (layer "F.Cu") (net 13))
 (segment (start 126.57625 128.635) (end 123.415 128.635) (width 0.2) (layer "F.Cu") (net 13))
 (segment (start 142.2 144.16) (end 163.03 144.16) (width 0.2) (layer "F.Cu") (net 13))
 (segment (start 141.98 58.54) (end 138 58.54) (width 0.2) (layer "F.Cu") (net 13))
 (segment (start 169.37 64.5) (end 167.05 62.18) (width 0.2) (layer "F.Cu") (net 13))
 (segment (start 167.05 62.18) (end 163.97 59.1) (width 0.2) (layer "F.Cu") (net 13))
 (segment (start 163.03 144.16) (end 169.37 137.82) (width 0.2) (layer "F.Cu") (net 13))
 (segment (start 123.415 128.635) (end 122.01 130.04) (width 0.2) (layer "F.Cu") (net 13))
 (segment (start 121.71 143) (end 122.87 144.16) (width 0.2) (layer "F.Cu") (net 13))
 (segment (start 122.87 144.16) (end 142.2 144.16) (width 0.2) (layer "F.Cu") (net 13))
 (via (at 163.97 59.01) (size 0.6) (drill 0.3) (layers "F.Cu" "B.Cu") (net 13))
 (via (at 141.98 58.54) (size 0.6) (drill 0.3) (layers "F.Cu" "B.Cu") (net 13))
 (segment (start 163.5 58.54) (end 163.97 59.01) (width 0.2) (layer "B.Cu") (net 13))
 (segment (start 141.98 58.54) (end 163.5 58.54) (width 0.2) (layer "B.Cu") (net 13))
 (segment (start 168.34 137.7) (end 168.34 65.34) (width 0.2) (layer "F.Cu") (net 5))
 (segment (start 141.06 142.39) (end 142.1 143.43) (width 0.2) (layer "F.Cu") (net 5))
 (segment (start 143.235 128.635) (end 140.95 130.92) (width 0.2) (layer "F.Cu") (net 5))
 (segment (start 168.34 65.34) (end 160.03 57.03) (width 0.2) (layer "F.Cu") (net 5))
 (segment (start 141.99 56) (end 138 56) (width 0.2) (layer "F.Cu") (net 5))
 (segment (start 141.06 131.03) (end 141.06 141.92) (width 0.2) (layer "F.Cu") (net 5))
 (segment (start 145.62625 128.635) (end 143.235 128.635) (width 0.2) (layer "F.Cu") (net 5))
 (segment (start 142.1 143.43) (end 162.61 143.43) (width 0.2) (layer "F.Cu") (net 5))
 (segment (start 141.06 141.92) (end 141.06 142.39) (width 0.2) (layer "F.Cu") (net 5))
 (segment (start 162.61 143.43) (end 168.34 137.7) (width 0.2) (layer "F.Cu") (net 5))
 (segment (start 140.95 130.92) (end 141.06 131.03) (width 0.2) (layer "F.Cu") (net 5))
 (via (at 141.99 56) (size 0.6) (drill 0.3) (layers "F.Cu" "B.Cu") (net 5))
 (via (at 160.03 57.03) (size 0.6) (drill 0.3) (layers "F.Cu" "B.Cu") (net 5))
 (segment (start 159 56) (end 141.99 56) (width 0.2) (layer "B.Cu") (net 5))
 (segment (start 160.03 57.03) (end 159 56) (width 0.2) (layer "B.Cu") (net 5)))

